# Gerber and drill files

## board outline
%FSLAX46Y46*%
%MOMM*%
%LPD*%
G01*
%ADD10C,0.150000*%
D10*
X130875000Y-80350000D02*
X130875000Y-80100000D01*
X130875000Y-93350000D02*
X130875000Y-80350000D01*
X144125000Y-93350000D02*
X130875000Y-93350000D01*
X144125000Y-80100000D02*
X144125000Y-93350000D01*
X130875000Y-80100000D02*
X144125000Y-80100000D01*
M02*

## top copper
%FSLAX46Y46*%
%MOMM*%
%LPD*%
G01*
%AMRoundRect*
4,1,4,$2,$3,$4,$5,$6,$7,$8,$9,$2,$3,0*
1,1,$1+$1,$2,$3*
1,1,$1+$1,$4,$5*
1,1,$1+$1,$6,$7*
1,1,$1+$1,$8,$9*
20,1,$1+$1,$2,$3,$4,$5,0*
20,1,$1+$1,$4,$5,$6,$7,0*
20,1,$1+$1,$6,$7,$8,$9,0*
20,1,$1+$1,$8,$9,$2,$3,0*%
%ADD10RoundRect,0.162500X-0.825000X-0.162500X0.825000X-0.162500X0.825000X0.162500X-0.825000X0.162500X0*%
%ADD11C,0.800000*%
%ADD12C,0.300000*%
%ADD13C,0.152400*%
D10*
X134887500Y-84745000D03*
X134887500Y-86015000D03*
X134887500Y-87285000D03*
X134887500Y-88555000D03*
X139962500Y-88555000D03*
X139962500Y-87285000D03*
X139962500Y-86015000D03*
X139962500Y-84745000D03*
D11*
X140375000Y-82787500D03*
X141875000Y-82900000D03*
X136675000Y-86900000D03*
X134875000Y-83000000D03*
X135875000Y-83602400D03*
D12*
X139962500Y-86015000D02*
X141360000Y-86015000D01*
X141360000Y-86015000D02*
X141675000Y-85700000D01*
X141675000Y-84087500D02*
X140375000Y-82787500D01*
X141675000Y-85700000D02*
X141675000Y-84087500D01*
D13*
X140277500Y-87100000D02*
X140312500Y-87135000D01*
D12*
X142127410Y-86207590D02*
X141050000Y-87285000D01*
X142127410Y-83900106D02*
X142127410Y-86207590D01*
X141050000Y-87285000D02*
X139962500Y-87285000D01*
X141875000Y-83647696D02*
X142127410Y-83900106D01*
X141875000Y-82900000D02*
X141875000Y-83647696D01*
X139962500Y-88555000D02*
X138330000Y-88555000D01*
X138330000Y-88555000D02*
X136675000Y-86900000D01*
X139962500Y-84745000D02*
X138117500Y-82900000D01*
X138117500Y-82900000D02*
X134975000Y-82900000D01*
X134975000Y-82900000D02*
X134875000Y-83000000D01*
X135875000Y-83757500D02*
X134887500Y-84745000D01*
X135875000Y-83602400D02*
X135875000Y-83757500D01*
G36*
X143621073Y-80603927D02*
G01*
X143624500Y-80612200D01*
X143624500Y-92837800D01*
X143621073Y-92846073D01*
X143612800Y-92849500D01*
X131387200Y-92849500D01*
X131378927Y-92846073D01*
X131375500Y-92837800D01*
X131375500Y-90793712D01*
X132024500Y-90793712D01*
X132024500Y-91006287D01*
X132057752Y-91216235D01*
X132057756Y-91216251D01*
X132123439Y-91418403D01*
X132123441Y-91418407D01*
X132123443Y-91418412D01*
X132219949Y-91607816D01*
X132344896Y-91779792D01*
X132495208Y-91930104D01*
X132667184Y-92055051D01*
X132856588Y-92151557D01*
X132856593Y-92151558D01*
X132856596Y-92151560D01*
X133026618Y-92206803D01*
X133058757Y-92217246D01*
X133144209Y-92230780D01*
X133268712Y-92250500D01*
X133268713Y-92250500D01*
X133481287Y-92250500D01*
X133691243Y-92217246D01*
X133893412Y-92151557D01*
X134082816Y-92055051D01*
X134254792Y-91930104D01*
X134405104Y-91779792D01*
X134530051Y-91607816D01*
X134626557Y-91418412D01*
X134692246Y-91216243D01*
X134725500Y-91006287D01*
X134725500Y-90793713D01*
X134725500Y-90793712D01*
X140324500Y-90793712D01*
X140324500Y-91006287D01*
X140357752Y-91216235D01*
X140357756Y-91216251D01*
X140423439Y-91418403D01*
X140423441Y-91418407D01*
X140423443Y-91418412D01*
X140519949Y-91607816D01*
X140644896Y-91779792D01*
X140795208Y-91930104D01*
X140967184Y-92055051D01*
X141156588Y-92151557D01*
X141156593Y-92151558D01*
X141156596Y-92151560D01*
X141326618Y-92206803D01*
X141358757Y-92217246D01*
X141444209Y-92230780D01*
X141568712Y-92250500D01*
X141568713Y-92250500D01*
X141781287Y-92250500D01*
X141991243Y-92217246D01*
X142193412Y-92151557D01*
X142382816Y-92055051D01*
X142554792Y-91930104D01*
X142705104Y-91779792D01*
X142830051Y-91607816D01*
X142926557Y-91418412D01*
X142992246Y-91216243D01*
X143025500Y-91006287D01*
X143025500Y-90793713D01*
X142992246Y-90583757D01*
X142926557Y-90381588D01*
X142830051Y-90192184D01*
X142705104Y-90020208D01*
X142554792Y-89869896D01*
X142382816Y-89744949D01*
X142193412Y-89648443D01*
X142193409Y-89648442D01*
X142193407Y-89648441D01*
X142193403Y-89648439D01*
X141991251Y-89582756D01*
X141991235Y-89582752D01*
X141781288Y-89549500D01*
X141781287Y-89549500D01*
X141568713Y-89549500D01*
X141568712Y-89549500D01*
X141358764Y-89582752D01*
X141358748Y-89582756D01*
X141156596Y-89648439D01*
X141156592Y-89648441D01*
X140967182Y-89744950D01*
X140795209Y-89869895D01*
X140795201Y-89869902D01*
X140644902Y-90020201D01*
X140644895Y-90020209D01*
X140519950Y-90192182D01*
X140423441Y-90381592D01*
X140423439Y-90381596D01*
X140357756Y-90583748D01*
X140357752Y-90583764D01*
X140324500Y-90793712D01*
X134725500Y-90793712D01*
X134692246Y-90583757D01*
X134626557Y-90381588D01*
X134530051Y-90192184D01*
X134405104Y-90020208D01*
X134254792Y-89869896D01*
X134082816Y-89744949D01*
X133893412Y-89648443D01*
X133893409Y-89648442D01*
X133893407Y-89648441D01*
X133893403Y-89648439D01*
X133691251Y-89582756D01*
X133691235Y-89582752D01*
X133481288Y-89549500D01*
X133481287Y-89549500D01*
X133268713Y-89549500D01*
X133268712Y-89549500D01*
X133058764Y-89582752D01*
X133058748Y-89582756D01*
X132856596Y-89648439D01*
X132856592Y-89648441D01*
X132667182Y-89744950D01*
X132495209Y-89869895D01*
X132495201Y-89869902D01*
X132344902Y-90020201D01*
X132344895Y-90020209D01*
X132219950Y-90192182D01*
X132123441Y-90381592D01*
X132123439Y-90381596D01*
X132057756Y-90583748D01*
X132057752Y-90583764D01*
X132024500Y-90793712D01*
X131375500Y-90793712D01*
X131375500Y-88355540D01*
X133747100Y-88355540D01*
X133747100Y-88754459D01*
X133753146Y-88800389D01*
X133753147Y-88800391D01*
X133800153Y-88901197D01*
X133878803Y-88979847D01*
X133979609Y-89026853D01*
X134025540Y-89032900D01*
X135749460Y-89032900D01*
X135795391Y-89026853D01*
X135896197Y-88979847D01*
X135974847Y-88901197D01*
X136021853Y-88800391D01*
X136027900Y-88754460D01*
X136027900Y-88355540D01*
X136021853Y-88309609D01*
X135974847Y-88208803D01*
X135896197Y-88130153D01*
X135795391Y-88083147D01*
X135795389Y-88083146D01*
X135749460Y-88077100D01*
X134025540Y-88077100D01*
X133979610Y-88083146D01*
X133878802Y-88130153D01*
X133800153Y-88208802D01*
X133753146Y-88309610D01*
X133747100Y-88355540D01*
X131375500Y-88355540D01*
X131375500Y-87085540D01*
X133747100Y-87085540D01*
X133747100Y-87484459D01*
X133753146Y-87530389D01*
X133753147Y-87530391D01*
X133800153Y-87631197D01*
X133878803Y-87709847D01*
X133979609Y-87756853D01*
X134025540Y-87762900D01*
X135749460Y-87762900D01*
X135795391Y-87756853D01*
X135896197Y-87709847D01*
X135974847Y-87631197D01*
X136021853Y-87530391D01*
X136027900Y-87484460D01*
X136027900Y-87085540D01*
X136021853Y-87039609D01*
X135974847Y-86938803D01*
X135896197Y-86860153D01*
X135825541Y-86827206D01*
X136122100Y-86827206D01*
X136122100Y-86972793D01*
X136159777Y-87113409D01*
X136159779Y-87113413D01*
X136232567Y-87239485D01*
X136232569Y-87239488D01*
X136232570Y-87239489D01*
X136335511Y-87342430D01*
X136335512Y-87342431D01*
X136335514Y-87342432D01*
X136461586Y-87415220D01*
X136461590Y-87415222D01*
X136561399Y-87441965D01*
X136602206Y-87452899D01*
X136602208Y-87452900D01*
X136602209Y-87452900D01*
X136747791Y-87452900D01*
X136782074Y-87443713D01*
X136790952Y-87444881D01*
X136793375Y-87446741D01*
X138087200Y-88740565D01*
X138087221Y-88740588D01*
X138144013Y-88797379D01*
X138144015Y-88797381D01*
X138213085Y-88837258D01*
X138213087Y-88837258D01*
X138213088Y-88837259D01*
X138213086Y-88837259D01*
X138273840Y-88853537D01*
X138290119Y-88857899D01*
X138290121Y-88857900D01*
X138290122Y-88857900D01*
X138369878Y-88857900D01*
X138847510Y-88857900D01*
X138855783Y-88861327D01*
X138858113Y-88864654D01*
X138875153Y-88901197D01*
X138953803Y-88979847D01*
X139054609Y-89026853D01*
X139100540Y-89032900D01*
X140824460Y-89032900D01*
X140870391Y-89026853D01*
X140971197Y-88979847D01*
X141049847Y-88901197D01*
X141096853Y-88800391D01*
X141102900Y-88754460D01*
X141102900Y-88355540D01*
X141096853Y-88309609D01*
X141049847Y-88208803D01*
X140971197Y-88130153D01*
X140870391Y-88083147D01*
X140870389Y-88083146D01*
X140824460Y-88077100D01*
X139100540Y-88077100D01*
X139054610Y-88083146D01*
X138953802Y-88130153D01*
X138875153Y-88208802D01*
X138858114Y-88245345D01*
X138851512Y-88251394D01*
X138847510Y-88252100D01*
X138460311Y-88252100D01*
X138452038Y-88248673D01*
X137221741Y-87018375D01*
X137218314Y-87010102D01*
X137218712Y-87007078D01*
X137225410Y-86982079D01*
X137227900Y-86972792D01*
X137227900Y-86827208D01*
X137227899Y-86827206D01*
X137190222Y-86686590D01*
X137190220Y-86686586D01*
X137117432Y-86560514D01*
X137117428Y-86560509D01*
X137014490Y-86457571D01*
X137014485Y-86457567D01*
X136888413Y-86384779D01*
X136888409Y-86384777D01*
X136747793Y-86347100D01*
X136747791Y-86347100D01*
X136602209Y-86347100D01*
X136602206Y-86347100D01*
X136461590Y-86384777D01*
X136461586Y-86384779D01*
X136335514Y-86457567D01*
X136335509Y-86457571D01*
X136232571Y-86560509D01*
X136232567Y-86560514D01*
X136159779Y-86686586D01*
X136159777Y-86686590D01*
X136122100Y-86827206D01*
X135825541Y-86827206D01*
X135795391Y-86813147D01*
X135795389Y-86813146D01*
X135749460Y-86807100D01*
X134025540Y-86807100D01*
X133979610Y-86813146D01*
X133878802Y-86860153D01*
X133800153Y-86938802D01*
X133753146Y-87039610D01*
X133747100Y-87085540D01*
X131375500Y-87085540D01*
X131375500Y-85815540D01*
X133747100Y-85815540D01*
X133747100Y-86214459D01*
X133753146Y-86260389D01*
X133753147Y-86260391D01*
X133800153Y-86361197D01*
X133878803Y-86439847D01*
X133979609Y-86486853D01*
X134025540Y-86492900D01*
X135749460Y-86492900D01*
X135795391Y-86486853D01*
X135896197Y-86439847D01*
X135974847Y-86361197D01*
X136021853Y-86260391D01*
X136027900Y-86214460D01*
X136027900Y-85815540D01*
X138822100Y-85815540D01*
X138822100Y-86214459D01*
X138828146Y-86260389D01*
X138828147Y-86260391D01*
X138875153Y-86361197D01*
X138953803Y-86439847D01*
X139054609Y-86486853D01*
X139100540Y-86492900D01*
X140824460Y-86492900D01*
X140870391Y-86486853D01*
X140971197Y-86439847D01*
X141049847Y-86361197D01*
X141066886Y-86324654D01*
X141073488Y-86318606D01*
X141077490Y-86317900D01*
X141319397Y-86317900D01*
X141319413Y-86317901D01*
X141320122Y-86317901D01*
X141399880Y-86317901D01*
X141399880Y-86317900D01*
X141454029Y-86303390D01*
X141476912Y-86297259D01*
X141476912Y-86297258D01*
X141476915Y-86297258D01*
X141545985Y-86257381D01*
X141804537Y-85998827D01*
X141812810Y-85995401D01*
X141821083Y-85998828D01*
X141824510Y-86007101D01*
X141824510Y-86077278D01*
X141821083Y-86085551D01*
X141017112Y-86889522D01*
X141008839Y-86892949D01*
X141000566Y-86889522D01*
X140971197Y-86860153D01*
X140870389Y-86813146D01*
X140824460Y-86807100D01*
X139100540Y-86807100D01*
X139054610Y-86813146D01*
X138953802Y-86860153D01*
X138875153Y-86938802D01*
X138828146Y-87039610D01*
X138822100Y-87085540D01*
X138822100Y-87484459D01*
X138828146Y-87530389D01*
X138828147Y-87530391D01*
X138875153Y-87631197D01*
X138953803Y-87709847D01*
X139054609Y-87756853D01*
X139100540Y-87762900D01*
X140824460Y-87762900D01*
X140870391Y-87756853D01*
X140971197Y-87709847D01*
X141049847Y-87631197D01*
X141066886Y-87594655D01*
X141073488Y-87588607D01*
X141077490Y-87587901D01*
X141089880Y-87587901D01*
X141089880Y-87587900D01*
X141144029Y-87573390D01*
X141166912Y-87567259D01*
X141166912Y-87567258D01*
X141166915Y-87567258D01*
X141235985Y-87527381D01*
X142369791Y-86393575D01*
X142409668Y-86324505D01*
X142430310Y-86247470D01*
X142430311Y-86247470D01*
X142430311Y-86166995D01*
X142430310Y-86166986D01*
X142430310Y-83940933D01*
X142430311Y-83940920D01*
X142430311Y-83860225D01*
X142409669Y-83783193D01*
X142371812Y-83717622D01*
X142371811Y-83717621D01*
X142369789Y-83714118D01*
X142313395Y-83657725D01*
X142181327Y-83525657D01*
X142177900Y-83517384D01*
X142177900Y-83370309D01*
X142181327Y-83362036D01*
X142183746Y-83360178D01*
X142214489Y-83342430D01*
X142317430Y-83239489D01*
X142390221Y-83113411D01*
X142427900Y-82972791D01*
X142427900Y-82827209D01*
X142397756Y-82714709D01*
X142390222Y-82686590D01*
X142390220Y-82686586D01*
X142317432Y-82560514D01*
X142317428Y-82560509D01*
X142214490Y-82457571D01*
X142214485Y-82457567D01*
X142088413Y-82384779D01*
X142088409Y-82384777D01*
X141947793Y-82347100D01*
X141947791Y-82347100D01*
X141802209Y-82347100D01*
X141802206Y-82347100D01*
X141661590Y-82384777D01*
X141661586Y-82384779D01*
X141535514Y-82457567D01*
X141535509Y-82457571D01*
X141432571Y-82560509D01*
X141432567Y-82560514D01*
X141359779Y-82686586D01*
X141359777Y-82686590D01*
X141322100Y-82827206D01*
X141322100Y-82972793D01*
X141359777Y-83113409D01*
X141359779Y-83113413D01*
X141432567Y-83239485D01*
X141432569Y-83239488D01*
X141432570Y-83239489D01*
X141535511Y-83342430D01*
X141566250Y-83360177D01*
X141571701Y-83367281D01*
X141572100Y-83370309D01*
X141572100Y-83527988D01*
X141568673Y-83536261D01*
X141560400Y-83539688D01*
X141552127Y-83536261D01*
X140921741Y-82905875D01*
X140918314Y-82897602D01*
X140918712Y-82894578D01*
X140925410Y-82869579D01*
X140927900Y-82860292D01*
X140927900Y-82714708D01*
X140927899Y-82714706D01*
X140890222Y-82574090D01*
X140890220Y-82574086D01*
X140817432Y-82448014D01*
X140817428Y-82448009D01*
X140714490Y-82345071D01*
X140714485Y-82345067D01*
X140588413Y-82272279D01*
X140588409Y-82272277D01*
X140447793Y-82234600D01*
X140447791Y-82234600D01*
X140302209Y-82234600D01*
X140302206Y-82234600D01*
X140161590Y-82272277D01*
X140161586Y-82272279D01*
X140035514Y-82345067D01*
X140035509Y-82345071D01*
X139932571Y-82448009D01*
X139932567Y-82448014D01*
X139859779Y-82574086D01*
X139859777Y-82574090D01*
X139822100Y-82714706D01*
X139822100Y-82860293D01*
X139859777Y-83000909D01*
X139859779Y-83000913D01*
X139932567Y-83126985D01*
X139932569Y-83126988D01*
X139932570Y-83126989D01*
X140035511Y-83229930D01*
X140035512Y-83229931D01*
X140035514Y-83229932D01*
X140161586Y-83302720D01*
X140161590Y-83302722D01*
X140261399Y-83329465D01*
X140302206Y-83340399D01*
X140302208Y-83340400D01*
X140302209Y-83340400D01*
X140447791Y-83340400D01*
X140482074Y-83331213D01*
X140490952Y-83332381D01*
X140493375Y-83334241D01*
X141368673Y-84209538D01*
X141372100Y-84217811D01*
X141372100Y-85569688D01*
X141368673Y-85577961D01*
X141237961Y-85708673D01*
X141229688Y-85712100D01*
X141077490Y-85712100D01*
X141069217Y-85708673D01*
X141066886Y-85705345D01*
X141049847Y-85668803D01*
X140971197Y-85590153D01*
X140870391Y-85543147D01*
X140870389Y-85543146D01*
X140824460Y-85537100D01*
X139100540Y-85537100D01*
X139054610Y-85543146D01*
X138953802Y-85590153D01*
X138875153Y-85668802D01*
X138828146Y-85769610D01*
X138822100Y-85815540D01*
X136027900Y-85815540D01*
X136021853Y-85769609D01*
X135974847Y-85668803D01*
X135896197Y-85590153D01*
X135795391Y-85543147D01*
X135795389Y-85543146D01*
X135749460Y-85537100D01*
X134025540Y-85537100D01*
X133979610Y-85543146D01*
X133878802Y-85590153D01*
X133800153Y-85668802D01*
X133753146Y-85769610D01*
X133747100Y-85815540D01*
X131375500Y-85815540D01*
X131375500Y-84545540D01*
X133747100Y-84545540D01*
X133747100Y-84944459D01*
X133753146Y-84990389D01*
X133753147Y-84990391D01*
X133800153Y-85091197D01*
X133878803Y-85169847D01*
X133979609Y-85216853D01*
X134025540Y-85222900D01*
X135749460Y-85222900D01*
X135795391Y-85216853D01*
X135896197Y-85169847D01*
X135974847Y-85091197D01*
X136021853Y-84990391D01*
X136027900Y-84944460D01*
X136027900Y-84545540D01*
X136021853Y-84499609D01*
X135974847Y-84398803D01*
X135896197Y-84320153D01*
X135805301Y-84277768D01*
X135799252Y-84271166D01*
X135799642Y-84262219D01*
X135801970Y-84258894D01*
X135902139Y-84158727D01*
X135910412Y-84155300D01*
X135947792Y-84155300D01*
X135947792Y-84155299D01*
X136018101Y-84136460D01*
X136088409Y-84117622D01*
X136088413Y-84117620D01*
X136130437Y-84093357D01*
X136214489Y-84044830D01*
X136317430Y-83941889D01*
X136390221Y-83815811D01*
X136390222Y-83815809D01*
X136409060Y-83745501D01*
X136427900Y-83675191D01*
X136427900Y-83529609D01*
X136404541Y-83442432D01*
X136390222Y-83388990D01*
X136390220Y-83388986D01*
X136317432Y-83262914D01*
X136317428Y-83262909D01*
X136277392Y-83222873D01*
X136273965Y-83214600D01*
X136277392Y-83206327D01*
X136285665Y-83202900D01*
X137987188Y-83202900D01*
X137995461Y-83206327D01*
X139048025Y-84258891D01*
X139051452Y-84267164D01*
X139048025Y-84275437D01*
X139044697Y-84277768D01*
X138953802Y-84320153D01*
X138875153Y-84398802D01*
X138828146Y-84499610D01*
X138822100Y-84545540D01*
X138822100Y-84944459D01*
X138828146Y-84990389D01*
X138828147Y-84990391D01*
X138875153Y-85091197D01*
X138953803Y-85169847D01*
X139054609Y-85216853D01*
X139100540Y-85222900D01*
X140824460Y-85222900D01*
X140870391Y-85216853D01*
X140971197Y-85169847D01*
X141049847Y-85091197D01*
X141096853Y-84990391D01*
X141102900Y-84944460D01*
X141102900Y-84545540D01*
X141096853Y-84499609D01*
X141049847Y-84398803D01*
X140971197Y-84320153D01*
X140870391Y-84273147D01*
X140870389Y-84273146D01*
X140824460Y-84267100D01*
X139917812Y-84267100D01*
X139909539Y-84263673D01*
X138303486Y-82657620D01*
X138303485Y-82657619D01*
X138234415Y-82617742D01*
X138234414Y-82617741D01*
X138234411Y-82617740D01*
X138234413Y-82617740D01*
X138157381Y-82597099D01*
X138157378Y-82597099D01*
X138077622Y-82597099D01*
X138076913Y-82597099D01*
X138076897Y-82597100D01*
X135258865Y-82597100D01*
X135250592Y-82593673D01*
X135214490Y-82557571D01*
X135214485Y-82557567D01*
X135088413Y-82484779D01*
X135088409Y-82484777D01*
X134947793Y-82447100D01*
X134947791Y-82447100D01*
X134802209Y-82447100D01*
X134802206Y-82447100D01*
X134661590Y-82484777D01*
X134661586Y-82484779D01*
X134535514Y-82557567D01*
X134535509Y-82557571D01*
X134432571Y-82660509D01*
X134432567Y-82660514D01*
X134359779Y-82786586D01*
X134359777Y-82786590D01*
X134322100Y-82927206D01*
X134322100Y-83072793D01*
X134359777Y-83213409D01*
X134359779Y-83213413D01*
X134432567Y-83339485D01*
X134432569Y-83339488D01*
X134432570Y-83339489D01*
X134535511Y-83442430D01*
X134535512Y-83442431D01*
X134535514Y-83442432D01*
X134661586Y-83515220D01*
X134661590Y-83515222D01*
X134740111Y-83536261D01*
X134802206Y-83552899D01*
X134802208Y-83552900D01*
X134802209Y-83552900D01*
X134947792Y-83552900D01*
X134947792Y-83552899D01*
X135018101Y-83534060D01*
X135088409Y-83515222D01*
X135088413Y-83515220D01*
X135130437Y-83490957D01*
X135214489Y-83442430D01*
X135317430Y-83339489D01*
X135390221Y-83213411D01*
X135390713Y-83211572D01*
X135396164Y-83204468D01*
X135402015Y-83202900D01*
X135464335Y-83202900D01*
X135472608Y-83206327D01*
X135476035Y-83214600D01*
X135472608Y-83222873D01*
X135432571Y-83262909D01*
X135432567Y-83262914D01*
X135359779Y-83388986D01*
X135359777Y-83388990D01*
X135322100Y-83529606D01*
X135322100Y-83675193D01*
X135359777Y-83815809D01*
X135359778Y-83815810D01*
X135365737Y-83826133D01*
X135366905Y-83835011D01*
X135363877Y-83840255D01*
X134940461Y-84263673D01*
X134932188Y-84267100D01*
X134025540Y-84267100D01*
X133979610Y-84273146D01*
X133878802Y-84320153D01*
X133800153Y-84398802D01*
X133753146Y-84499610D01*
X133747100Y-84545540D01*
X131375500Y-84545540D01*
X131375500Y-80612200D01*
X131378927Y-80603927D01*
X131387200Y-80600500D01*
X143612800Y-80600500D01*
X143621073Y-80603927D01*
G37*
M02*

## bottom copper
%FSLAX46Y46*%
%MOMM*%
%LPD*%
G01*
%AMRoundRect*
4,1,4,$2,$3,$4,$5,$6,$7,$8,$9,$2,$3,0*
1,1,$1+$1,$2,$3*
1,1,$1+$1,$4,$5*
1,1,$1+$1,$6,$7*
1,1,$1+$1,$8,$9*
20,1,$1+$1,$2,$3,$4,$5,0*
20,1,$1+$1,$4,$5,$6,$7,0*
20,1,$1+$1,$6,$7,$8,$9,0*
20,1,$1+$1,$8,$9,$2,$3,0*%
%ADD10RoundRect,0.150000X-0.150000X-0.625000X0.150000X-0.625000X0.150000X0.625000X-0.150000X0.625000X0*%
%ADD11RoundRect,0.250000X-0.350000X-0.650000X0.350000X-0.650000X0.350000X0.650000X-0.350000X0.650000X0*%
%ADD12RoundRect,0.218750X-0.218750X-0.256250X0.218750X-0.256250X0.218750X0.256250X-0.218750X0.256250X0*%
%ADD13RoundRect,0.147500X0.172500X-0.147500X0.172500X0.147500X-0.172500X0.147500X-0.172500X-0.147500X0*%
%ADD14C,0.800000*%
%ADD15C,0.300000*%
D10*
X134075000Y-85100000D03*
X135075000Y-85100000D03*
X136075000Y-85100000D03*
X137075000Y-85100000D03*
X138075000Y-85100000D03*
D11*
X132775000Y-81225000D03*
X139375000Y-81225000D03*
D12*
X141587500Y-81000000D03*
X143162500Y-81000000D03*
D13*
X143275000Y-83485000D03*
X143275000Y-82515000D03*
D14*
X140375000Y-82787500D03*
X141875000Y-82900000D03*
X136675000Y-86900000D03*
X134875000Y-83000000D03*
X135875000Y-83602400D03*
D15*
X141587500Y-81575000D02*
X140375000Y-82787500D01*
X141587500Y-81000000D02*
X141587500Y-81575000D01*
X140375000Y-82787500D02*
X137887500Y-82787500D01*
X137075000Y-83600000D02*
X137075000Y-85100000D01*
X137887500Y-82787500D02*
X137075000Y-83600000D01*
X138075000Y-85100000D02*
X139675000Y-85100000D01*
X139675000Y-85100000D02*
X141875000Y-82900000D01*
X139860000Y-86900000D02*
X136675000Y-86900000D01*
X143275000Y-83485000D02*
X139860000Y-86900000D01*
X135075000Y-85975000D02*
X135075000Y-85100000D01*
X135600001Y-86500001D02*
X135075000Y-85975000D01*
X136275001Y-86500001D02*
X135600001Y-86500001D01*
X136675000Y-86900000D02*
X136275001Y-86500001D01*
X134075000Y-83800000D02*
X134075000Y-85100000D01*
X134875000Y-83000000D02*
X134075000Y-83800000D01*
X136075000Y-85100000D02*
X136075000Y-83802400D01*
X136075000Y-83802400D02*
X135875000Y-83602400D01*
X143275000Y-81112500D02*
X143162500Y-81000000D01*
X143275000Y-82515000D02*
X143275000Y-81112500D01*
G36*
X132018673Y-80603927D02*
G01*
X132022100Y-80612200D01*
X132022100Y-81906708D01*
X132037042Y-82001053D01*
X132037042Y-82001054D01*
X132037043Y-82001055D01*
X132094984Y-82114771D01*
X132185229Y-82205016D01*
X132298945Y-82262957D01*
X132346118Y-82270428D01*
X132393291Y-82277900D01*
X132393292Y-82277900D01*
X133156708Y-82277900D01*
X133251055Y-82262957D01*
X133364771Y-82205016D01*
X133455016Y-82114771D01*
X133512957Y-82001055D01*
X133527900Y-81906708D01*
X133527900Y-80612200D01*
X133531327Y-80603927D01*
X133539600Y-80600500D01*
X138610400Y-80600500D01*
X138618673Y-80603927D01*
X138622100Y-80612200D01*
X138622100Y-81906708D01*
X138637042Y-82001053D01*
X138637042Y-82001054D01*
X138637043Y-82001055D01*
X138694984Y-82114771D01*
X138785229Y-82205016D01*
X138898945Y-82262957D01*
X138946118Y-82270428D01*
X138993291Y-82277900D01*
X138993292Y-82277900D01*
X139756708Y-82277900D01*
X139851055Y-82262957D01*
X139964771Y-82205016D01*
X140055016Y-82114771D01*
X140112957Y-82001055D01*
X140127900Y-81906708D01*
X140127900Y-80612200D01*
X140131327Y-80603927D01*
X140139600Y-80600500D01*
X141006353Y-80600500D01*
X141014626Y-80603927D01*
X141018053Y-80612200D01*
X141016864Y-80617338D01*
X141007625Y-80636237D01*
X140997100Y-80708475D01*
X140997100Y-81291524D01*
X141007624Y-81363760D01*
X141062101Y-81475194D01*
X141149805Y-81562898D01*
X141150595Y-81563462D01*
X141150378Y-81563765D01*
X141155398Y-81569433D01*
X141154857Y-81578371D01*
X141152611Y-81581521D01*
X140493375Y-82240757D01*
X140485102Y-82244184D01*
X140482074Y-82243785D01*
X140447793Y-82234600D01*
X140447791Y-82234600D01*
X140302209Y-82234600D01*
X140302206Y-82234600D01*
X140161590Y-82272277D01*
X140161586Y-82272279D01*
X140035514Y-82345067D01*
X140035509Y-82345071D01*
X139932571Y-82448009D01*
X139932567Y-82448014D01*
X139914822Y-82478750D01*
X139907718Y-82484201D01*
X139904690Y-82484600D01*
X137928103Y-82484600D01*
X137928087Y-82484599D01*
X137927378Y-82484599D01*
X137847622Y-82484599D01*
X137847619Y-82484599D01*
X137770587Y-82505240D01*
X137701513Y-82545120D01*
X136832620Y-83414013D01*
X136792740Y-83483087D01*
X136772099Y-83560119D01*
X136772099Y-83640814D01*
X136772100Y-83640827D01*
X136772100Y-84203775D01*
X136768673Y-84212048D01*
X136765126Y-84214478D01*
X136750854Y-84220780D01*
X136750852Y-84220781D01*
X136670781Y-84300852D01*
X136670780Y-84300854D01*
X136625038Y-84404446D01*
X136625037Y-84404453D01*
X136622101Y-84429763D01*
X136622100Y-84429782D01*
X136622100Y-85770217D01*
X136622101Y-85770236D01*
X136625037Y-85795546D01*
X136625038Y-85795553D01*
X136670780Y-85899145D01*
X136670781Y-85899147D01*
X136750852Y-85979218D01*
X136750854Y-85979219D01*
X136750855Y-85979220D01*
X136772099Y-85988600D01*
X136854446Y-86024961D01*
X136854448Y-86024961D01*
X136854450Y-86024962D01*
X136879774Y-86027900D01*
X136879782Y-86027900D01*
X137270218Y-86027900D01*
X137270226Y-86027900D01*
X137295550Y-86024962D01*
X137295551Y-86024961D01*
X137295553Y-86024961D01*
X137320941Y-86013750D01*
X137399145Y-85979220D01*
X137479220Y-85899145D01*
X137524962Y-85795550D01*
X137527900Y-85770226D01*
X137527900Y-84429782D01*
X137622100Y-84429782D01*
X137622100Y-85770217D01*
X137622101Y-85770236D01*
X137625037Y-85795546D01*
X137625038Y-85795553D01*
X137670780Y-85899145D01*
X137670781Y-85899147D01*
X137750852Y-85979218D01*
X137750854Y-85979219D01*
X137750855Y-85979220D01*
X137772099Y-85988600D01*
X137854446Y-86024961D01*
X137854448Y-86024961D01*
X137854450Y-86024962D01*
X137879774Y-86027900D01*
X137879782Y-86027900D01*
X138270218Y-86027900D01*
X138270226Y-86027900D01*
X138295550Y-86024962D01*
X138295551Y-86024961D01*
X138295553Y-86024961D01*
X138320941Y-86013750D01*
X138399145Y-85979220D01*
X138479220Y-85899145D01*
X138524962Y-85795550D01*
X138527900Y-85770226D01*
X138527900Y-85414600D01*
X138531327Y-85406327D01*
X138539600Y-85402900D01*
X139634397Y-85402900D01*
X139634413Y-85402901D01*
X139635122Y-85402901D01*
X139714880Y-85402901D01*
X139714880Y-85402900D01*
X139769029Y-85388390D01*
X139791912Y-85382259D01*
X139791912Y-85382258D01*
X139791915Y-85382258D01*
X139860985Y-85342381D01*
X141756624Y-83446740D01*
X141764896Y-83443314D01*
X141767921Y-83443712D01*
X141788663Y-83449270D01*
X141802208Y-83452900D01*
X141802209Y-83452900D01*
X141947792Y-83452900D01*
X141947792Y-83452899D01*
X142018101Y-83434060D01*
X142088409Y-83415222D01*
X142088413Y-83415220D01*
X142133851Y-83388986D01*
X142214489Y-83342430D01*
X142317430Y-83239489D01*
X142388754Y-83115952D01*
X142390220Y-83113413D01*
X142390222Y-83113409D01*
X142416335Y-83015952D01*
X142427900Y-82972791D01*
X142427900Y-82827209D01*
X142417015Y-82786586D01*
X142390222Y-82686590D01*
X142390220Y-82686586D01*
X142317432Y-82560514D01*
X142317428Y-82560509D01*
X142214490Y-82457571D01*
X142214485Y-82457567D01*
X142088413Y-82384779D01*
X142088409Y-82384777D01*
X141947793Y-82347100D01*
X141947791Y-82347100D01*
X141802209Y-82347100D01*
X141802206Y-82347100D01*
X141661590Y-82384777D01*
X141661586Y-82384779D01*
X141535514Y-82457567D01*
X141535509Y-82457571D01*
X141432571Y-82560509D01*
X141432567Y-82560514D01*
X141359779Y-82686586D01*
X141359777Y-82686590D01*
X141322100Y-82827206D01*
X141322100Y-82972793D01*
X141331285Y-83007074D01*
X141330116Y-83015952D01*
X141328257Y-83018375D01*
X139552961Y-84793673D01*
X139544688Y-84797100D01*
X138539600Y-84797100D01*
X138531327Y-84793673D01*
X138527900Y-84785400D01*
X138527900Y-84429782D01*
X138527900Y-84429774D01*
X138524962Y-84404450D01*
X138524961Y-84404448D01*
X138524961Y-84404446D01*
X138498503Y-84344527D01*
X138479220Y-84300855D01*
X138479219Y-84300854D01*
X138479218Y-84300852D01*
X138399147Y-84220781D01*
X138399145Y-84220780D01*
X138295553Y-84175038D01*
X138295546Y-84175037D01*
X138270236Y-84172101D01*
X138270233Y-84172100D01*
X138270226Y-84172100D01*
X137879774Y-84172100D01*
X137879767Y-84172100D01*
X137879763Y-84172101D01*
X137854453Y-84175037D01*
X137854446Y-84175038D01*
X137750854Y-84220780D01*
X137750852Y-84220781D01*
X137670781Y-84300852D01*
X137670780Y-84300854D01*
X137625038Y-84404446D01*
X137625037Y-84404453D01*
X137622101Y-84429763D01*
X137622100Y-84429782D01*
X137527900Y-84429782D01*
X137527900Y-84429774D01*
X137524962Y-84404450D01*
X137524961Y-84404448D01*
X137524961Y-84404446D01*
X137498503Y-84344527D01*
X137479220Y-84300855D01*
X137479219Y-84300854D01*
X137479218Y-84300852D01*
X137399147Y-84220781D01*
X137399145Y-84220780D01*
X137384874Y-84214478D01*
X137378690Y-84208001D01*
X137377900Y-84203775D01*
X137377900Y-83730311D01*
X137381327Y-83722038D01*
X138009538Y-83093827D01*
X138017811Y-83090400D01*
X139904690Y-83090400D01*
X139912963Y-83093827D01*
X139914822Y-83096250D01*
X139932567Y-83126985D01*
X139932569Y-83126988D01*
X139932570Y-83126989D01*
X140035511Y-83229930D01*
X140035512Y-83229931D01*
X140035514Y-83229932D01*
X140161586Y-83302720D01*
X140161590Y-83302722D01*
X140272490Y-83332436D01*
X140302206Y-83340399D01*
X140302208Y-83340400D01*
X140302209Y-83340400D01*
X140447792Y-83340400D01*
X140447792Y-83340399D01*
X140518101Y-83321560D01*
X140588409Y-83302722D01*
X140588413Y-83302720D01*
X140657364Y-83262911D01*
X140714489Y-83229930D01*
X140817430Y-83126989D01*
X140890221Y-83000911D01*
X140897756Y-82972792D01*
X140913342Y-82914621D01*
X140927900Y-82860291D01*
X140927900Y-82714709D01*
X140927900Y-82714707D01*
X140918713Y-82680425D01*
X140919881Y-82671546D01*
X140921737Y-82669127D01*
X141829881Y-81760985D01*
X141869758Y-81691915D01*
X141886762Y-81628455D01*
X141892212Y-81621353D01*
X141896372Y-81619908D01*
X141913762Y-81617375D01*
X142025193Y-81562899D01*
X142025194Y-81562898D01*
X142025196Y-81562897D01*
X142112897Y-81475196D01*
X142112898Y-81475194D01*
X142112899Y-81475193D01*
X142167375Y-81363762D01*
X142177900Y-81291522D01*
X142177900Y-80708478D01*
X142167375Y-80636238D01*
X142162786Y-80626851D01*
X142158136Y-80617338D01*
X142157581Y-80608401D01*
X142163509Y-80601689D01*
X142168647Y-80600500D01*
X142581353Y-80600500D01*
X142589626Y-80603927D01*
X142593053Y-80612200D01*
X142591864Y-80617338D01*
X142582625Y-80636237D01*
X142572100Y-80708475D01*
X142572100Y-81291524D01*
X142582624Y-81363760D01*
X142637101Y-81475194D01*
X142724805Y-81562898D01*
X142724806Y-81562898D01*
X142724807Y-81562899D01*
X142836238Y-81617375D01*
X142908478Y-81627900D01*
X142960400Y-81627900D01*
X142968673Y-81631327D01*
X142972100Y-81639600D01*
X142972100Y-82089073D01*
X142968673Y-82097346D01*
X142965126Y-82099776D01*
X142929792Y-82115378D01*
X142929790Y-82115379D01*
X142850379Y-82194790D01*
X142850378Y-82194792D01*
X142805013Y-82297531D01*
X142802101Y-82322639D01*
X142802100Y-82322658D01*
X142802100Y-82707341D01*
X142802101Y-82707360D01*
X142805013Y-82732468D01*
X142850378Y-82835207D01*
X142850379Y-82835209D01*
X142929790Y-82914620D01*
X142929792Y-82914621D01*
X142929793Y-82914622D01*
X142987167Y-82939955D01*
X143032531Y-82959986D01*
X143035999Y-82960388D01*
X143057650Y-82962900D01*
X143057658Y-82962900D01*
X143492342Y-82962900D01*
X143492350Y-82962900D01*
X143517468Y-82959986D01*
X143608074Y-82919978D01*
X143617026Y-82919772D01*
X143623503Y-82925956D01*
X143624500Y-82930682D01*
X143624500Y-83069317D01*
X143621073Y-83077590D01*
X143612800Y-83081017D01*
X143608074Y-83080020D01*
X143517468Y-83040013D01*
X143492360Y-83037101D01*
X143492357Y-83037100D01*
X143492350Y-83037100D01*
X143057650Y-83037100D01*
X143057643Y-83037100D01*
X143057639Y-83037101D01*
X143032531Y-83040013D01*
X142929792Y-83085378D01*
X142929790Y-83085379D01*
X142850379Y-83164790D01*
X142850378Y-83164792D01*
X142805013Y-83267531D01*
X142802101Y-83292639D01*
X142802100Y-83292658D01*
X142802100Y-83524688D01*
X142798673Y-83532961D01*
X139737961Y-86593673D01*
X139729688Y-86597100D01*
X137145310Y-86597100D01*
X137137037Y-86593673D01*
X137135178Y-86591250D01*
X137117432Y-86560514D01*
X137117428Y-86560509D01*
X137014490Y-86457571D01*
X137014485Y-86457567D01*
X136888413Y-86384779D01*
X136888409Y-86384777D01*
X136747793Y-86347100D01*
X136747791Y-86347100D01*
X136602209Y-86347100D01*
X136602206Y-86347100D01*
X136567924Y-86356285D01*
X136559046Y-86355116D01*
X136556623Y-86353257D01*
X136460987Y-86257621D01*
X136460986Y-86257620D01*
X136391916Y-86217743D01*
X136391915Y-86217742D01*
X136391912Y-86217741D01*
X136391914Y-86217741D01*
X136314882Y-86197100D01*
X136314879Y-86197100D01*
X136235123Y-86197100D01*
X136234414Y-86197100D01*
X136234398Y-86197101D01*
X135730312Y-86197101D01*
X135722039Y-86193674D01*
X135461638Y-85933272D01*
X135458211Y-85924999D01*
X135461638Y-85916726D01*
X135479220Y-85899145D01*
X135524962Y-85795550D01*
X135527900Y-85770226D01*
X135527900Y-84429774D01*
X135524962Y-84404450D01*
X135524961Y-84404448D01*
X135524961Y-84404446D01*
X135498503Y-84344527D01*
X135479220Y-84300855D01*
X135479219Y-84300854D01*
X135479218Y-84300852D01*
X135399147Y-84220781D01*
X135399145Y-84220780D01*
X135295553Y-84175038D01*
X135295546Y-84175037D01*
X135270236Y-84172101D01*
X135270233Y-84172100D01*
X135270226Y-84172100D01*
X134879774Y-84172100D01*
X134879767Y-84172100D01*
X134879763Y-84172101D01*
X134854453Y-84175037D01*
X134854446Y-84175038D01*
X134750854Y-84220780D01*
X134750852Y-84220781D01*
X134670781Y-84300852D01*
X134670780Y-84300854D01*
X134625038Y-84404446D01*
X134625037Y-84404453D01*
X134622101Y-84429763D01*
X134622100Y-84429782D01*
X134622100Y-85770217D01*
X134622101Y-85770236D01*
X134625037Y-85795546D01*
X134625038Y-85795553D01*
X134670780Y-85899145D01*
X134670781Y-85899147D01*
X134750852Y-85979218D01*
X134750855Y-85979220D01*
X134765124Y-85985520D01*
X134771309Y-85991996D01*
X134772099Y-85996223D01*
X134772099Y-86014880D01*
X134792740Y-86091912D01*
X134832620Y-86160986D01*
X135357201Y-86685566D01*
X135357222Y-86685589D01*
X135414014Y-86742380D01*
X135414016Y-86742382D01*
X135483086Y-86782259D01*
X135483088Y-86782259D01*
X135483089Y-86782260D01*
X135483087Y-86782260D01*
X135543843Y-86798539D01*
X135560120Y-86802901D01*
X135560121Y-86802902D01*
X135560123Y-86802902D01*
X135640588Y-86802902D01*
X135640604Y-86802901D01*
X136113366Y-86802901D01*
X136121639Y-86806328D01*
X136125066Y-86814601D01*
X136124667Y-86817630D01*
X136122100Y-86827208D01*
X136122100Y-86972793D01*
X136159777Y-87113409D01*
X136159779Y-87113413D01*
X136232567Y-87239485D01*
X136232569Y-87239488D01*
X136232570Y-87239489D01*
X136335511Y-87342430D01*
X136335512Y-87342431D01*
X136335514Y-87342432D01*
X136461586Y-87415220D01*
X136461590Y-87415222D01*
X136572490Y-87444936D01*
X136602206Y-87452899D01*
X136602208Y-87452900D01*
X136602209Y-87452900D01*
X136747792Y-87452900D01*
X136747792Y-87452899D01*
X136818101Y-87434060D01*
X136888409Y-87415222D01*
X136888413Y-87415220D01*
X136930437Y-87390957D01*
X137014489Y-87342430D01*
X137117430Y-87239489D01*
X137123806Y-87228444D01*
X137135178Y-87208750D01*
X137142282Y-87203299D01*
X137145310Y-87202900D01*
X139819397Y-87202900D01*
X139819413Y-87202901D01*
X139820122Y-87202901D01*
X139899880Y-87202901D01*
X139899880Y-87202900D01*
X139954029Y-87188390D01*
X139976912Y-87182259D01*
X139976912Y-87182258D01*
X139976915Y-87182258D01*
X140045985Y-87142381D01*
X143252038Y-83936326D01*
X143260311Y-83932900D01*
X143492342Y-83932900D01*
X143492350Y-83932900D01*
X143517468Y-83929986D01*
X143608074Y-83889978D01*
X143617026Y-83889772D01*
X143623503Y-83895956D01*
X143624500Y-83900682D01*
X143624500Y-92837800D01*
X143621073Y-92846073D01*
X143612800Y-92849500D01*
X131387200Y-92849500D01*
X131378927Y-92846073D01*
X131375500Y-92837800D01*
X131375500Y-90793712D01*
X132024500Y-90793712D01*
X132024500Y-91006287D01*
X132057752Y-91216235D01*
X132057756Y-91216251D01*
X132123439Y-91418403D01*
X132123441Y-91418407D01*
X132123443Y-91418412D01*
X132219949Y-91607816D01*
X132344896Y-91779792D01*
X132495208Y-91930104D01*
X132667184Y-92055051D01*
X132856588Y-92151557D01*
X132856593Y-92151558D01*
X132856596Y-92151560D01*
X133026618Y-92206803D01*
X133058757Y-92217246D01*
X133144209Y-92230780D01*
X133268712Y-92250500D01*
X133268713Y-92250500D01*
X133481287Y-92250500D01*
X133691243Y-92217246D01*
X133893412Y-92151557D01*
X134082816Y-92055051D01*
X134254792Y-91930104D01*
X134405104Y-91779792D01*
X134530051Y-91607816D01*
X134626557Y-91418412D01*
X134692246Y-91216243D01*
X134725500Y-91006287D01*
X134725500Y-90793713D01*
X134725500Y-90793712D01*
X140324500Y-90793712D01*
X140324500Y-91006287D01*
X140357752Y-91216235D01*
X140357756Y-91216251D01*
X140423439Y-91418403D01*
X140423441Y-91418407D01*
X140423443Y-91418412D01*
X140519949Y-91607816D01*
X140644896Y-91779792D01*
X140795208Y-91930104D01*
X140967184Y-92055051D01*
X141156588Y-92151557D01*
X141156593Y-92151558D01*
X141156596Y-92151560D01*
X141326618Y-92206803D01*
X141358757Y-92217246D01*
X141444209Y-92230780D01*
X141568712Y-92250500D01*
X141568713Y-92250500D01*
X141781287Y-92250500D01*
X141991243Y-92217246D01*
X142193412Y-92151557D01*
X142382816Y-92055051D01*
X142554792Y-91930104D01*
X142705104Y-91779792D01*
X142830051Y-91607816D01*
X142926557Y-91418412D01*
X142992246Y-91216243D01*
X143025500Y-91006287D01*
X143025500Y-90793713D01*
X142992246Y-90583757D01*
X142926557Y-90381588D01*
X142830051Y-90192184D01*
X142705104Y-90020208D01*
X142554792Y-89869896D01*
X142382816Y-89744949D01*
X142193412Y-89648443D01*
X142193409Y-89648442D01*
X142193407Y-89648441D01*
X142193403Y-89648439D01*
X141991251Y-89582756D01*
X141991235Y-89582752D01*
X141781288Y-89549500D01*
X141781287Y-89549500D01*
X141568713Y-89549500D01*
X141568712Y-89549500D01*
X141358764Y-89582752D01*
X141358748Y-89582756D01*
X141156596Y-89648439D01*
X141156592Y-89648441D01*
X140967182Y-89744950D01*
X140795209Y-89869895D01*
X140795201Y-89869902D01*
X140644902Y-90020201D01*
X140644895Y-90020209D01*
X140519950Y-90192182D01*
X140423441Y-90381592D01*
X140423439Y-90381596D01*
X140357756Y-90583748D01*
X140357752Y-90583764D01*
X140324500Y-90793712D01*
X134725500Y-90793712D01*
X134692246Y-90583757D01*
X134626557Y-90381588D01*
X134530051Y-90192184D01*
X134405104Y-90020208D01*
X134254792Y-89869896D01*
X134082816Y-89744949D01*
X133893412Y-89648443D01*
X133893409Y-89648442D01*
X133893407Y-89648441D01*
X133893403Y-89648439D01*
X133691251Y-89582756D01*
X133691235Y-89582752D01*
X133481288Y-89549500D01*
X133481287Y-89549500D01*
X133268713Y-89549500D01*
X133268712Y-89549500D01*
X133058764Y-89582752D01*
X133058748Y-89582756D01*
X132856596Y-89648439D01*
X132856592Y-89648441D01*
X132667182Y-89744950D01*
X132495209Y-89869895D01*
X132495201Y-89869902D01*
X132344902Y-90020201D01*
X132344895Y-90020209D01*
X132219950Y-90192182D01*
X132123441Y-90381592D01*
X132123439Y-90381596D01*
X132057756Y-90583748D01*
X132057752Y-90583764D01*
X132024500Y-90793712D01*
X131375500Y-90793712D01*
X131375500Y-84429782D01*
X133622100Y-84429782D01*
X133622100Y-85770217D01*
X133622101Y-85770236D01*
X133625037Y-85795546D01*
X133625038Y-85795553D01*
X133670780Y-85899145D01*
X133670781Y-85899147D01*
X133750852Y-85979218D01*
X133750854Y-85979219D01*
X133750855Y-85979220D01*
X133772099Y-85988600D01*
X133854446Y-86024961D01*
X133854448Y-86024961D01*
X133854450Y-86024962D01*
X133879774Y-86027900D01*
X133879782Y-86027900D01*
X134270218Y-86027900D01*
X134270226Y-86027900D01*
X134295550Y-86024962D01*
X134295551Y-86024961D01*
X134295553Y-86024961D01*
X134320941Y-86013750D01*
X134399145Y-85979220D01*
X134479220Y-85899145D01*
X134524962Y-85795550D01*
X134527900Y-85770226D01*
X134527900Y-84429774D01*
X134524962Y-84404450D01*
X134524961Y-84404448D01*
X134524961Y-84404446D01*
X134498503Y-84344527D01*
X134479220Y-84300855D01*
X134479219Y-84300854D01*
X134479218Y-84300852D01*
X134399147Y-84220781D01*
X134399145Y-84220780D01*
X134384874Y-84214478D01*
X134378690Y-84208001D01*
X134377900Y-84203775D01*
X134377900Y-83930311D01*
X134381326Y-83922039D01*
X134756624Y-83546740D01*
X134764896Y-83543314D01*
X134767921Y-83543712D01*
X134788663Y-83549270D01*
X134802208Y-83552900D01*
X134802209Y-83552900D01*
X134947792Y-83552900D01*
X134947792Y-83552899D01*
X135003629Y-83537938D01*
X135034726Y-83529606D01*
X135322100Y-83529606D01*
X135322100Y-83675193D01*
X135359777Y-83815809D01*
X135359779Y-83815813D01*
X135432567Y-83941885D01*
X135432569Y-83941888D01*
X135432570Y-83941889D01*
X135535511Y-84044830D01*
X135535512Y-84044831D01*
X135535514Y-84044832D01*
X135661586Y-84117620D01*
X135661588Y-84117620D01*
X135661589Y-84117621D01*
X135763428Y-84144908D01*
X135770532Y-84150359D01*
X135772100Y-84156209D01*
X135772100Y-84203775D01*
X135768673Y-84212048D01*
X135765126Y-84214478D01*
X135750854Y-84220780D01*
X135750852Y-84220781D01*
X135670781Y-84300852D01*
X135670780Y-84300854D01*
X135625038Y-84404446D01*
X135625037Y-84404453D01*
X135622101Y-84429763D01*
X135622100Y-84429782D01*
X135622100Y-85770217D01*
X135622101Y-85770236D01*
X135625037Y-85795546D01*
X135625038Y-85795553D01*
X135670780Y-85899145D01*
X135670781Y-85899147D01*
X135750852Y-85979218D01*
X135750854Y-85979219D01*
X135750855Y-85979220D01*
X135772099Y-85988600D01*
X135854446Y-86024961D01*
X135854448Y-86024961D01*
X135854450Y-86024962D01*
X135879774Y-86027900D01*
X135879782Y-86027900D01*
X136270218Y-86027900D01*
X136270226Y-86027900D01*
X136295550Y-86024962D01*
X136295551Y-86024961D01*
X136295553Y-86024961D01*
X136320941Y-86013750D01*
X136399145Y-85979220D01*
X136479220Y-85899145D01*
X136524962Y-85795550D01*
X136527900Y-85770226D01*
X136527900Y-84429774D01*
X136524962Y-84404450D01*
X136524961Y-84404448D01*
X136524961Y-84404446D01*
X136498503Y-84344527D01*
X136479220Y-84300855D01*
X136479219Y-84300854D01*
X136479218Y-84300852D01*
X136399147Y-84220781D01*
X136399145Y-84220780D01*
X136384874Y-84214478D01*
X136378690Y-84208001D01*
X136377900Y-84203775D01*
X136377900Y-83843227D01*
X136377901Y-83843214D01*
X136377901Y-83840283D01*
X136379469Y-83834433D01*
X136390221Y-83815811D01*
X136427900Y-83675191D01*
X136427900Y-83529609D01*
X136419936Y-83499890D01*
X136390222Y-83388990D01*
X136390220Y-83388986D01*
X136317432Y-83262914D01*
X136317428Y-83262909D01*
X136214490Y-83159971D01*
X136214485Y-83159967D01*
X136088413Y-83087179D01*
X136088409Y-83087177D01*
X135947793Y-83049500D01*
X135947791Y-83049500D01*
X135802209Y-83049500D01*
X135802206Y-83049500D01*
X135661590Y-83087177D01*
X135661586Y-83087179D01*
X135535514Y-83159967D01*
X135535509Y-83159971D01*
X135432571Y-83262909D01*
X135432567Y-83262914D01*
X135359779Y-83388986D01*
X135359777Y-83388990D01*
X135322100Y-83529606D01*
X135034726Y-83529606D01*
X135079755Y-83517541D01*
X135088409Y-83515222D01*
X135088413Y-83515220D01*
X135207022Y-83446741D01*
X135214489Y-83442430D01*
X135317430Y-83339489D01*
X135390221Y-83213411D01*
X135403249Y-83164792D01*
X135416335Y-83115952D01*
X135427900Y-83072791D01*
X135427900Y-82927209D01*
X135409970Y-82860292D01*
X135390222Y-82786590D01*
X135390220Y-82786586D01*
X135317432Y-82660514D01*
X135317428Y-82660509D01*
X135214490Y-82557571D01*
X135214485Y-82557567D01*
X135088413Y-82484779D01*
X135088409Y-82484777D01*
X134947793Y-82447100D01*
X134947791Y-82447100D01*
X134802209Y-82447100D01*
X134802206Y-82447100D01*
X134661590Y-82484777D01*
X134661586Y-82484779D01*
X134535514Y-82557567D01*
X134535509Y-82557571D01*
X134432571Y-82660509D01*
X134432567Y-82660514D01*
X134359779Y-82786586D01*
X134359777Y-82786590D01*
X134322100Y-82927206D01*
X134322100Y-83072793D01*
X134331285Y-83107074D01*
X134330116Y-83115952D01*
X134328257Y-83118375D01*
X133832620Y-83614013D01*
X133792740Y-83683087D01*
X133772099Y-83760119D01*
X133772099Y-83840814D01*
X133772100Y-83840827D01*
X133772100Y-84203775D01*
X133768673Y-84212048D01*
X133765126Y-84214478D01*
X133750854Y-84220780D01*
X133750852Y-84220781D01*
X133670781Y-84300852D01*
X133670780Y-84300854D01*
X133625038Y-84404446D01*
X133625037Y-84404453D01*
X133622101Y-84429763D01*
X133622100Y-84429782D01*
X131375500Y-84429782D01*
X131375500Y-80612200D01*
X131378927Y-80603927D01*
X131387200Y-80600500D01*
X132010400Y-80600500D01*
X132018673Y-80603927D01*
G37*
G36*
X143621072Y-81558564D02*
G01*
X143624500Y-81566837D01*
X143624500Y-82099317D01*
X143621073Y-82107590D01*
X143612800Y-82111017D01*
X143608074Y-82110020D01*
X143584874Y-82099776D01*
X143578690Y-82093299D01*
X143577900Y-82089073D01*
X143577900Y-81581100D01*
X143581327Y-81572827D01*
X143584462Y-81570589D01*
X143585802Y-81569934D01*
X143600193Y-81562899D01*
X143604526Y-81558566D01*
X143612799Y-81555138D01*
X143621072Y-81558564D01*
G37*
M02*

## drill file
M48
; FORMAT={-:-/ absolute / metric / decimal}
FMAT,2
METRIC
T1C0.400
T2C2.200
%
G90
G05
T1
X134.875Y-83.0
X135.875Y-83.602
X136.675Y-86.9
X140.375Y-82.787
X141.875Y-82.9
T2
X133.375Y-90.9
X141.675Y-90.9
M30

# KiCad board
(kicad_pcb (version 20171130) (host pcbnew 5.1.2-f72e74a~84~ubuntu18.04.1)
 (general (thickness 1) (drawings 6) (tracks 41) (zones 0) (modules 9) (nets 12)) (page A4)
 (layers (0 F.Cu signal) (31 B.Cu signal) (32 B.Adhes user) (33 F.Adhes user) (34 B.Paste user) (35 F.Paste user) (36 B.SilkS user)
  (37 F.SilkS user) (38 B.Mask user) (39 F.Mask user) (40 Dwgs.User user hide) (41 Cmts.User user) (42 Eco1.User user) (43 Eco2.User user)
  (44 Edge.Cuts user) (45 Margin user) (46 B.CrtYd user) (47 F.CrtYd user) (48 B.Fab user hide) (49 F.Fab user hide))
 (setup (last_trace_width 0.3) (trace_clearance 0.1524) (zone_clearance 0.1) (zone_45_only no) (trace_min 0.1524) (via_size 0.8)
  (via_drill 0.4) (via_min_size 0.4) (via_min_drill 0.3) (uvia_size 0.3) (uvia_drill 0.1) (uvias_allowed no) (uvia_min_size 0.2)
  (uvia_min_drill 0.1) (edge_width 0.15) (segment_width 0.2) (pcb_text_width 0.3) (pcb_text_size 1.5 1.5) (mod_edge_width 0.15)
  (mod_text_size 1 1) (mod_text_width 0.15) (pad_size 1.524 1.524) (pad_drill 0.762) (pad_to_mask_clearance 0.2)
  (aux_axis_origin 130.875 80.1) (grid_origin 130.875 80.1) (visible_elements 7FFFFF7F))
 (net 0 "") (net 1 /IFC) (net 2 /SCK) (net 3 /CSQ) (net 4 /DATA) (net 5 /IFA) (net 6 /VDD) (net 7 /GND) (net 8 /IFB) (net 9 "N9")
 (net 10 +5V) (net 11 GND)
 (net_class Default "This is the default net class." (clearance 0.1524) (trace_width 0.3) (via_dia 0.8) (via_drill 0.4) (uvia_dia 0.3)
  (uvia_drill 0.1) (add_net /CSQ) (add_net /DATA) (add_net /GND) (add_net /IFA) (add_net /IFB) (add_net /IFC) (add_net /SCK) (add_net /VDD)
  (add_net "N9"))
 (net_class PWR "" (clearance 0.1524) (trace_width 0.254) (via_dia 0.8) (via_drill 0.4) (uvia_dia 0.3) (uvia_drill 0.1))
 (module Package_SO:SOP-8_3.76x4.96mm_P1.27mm (layer F.Cu) (at 137.425 86.65)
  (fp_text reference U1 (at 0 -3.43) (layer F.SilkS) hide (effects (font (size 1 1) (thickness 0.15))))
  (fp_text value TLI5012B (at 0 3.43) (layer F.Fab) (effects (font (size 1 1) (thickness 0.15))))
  (pad 1 smd roundrect (at -2.5375 -1.905) (size 1.975 0.65) (layers F.Cu F.Paste F.Mask) (roundrect_rratio 0.25) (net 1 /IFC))
  (pad 2 smd roundrect (at -2.5375 -0.635) (size 1.975 0.65) (layers F.Cu F.Paste F.Mask) (roundrect_rratio 0.25) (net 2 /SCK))
  (pad 3 smd roundrect (at -2.5375 0.635) (size 1.975 0.65) (layers F.Cu F.Paste F.Mask) (roundrect_rratio 0.25) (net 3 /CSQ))
  (pad 4 smd roundrect (at -2.5375 1.905) (size 1.975 0.65) (layers F.Cu F.Paste F.Mask) (roundrect_rratio 0.25) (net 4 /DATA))
  (pad 5 smd roundrect (at 2.5375 1.905) (size 1.975 0.65) (layers F.Cu F.Paste F.Mask) (roundrect_rratio 0.25) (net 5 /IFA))
  (pad 6 smd roundrect (at 2.5375 0.635) (size 1.975 0.65) (layers F.Cu F.Paste F.Mask) (roundrect_rratio 0.25) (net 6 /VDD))
  (pad 7 smd roundrect (at 2.5375 -0.635) (size 1.975 0.65) (layers F.Cu F.Paste F.Mask) (roundrect_rratio 0.25) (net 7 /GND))
  (pad 8 smd roundrect (at 2.5375 -1.905) (size 1.975 0.65) (layers F.Cu F.Paste F.Mask) (roundrect_rratio 0.25) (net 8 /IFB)))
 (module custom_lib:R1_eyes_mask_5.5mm (layer B.Cu) (at 137.575 90.3 180)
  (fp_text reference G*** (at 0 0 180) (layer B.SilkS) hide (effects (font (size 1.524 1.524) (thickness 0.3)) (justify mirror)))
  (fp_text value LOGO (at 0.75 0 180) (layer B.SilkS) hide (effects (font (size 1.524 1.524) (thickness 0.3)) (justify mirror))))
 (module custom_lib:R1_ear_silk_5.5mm (layer B.Cu) (at 137.575 90.3 180)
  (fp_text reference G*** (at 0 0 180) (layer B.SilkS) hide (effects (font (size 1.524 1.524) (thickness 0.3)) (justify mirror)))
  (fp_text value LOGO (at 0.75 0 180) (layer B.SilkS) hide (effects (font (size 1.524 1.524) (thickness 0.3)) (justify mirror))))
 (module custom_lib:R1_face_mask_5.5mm (layer B.Cu) (at 137.575 90.3 180)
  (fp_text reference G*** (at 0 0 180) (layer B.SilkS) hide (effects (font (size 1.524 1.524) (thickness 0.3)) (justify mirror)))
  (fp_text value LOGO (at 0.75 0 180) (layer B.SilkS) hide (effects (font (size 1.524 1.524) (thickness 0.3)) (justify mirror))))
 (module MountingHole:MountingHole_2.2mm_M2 (layer F.Cu) (at 133.375 90.9)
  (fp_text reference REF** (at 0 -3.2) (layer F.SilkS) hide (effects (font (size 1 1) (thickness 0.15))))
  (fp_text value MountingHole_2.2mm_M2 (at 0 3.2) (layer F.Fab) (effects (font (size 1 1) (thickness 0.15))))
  (pad 1 np_thru_hole circle (at 0 0) (size 2.2 2.2) (drill 2.2) (layers *.Cu *.Mask)))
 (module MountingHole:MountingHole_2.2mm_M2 (layer F.Cu) (at 141.675 90.9)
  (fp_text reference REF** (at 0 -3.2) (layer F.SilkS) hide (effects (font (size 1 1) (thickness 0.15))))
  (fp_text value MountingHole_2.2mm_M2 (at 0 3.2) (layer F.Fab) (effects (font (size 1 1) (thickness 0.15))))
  (pad 1 np_thru_hole circle (at 0 0) (size 2.2 2.2) (drill 2.2) (layers *.Cu *.Mask)))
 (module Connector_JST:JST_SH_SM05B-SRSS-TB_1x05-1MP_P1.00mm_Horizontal (layer B.Cu) (at 136.075 83.1)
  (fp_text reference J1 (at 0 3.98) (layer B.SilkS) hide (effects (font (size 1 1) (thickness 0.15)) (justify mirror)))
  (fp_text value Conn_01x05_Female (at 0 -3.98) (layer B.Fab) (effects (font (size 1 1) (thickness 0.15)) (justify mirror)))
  (pad 1 smd roundrect (at -2 2) (size 0.6 1.55) (layers B.Cu B.Paste B.Mask) (roundrect_rratio 0.25) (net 8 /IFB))
  (pad 2 smd roundrect (at -1 2) (size 0.6 1.55) (layers B.Cu B.Paste B.Mask) (roundrect_rratio 0.25) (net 5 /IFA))
  (pad 3 smd roundrect (at 0 2) (size 0.6 1.55) (layers B.Cu B.Paste B.Mask) (roundrect_rratio 0.25) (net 1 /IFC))
  (pad 4 smd roundrect (at 1 2) (size 0.6 1.55) (layers B.Cu B.Paste B.Mask) (roundrect_rratio 0.25) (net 7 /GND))
  (pad 5 smd roundrect (at 2 2) (size 0.6 1.55) (layers B.Cu B.Paste B.Mask) (roundrect_rratio 0.25) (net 6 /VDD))
  (pad MP smd roundrect (at -3.3 -1.875) (size 1.2 1.8) (layers B.Cu B.Paste B.Mask) (roundrect_rratio 0.208333))
  (pad MP smd roundrect (at 3.3 -1.875) (size 1.2 1.8) (layers B.Cu B.Paste B.Mask) (roundrect_rratio 0.208333)))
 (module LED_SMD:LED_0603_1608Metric (layer B.Cu) (at 142.375 81)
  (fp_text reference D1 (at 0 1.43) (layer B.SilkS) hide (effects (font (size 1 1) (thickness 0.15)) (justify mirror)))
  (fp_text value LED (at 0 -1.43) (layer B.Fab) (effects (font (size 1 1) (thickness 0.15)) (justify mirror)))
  (pad 1 smd roundrect (at -0.7875 0) (size 0.875 0.95) (layers B.Cu B.Paste B.Mask) (roundrect_rratio 0.25) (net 7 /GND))
  (pad 2 smd roundrect (at 0.7875 0) (size 0.875 0.95) (layers B.Cu B.Paste B.Mask) (roundrect_rratio 0.25) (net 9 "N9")))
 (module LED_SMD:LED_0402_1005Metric (layer B.Cu) (at 143.275 83 90)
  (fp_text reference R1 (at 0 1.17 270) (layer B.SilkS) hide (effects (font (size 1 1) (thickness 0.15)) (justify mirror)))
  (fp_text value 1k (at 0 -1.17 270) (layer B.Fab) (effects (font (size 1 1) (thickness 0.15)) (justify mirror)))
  (pad 1 smd roundrect (at -0.485 0 90) (size 0.59 0.64) (layers B.Cu B.Paste B.Mask) (roundrect_rratio 0.25) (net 5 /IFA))
  (pad 2 smd roundrect (at 0.485 0 90) (size 0.59 0.64) (layers B.Cu B.Paste B.Mask) (roundrect_rratio 0.25) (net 9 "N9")))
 (gr_line (start 130.875 80.35) (end 130.875 80.1) (layer Edge.Cuts) (width 0.15))
 (gr_line (start 130.875 93.35) (end 130.875 80.35) (layer Edge.Cuts) (width 0.15))
 (gr_line (start 144.125 93.35) (end 130.875 93.35) (layer Edge.Cuts) (width 0.15))
 (gr_line (start 144.125 80.1) (end 144.125 93.35) (layer Edge.Cuts) (width 0.15))
 (gr_line (start 130.875 80.1) (end 144.125 80.1) (angle 90) (layer Edge.Cuts) (width 0.15))
 (segment (start 141.5875 81.575) (end 140.375 82.7875) (width 0.3) (layer B.Cu) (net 7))
 (segment (start 141.5875 81) (end 141.5875 81.575) (width 0.3) (layer B.Cu) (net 7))
 (segment (start 140.375 82.7875) (end 137.8875 82.7875) (width 0.3) (layer B.Cu) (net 7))
 (segment (start 137.075 83.6) (end 137.075 85.1) (width 0.3) (layer B.Cu) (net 7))
 (segment (start 137.8875 82.7875) (end 137.075 83.6) (width 0.3) (layer B.Cu) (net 7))
 (via (at 140.375 82.7875) (size 0.8) (drill 0.4) (layers F.Cu B.Cu) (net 7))
 (segment (start 139.9625 86.015) (end 141.36 86.015) (width 0.3) (layer F.Cu) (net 7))
 (segment (start 141.36 86.015) (end 141.675 85.7) (width 0.3) (layer F.Cu) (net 7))
 (segment (start 141.675 84.0875) (end 140.375 82.7875) (width 0.3) (layer F.Cu) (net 7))
 (segment (start 141.675 85.7) (end 141.675 84.0875) (width 0.3) (layer F.Cu) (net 7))
 (segment (start 140.2775 87.1) (end 140.3125 87.135) (width 0.1524) (layer F.Cu) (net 6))
 (via (at 141.875 82.9) (size 0.8) (drill 0.4) (layers F.Cu B.Cu) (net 6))
 (segment (start 138.075 85.1) (end 139.675 85.1) (width 0.3) (layer B.Cu) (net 6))
 (segment (start 139.675 85.1) (end 141.875 82.9) (width 0.3) (layer B.Cu) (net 6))
 (segment (start 142.12741 86.20759) (end 141.05 87.285) (width 0.3) (layer F.Cu) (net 6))
 (segment (start 142.12741 83.900106) (end 142.12741 86.20759) (width 0.3) (layer F.Cu) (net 6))
 (segment (start 141.05 87.285) (end 139.9625 87.285) (width 0.3) (layer F.Cu) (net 6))
 (segment (start 141.875 83.647696) (end 142.12741 83.900106) (width 0.3) (layer F.Cu) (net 6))
 (segment (start 141.875 82.9) (end 141.875 83.647696) (width 0.3) (layer F.Cu) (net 6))
 (via (at 136.675 86.9) (size 0.8) (drill 0.4) (layers F.Cu B.Cu) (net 5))
 (segment (start 139.9625 88.555) (end 138.33 88.555) (width 0.3) (layer F.Cu) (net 5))
 (segment (start 138.33 88.555) (end 136.675 86.9) (width 0.3) (layer F.Cu) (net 5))
 (segment (start 139.86 86.9) (end 136.675 86.9) (width 0.3) (layer B.Cu) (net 5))
 (segment (start 143.275 83.485) (end 139.86 86.9) (width 0.3) (layer B.Cu) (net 5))
 (segment (start 135.075 85.975) (end 135.075 85.1) (width 0.3) (layer B.Cu) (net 5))
 (segment (start 135.600001 86.500001) (end 135.075 85.975) (width 0.3) (layer B.Cu) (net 5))
 (segment (start 136.275001 86.500001) (end 135.600001 86.500001) (width 0.3) (layer B.Cu) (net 5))
 (segment (start 136.675 86.9) (end 136.275001 86.500001) (width 0.3) (layer B.Cu) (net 5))
 (segment (start 139.9625 84.745) (end 138.1175 82.9) (width 0.3) (layer F.Cu) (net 8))
 (segment (start 138.1175 82.9) (end 134.975 82.9) (width 0.3) (layer F.Cu) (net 8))
 (via (at 134.875 83) (size 0.8) (drill 0.4) (layers F.Cu B.Cu) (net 8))
 (segment (start 134.975 82.9) (end 134.875 83) (width 0.3) (layer F.Cu) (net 8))
 (segment (start 134.075 83.8) (end 134.075 85.1) (width 0.3) (layer B.Cu) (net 8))
 (segment (start 134.875 83) (end 134.075 83.8) (width 0.3) (layer B.Cu) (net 8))
 (via (at 135.875 83.6024) (size 0.8) (drill 0.4) (layers F.Cu B.Cu) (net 1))
 (segment (start 136.075 85.1) (end 136.075 83.8024) (width 0.3) (layer B.Cu) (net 1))
 (segment (start 136.075 83.8024) (end 135.875 83.6024) (width 0.3) (layer B.Cu) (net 1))
 (segment (start 135.875 83.7575) (end 134.8875 84.745) (width 0.3) (layer F.Cu) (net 1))
 (segment (start 135.875 83.6024) (end 135.875 83.7575) (width 0.3) (layer F.Cu) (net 1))
 (segment (start 143.275 81.1125) (end 143.1625 81) (width 0.3) (layer B.Cu) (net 9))
 (segment (start 143.275 82.515) (end 143.275 81.1125) (width 0.3) (layer B.Cu) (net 9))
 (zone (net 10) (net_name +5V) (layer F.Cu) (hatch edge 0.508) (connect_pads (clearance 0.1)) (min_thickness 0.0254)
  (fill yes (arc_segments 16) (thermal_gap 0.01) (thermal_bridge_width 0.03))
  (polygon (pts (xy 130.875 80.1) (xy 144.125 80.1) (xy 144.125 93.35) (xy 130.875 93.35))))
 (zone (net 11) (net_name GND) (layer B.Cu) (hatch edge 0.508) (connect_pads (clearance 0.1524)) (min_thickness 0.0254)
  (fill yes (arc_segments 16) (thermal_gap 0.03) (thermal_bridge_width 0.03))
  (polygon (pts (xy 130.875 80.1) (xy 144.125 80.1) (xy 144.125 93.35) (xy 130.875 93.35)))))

